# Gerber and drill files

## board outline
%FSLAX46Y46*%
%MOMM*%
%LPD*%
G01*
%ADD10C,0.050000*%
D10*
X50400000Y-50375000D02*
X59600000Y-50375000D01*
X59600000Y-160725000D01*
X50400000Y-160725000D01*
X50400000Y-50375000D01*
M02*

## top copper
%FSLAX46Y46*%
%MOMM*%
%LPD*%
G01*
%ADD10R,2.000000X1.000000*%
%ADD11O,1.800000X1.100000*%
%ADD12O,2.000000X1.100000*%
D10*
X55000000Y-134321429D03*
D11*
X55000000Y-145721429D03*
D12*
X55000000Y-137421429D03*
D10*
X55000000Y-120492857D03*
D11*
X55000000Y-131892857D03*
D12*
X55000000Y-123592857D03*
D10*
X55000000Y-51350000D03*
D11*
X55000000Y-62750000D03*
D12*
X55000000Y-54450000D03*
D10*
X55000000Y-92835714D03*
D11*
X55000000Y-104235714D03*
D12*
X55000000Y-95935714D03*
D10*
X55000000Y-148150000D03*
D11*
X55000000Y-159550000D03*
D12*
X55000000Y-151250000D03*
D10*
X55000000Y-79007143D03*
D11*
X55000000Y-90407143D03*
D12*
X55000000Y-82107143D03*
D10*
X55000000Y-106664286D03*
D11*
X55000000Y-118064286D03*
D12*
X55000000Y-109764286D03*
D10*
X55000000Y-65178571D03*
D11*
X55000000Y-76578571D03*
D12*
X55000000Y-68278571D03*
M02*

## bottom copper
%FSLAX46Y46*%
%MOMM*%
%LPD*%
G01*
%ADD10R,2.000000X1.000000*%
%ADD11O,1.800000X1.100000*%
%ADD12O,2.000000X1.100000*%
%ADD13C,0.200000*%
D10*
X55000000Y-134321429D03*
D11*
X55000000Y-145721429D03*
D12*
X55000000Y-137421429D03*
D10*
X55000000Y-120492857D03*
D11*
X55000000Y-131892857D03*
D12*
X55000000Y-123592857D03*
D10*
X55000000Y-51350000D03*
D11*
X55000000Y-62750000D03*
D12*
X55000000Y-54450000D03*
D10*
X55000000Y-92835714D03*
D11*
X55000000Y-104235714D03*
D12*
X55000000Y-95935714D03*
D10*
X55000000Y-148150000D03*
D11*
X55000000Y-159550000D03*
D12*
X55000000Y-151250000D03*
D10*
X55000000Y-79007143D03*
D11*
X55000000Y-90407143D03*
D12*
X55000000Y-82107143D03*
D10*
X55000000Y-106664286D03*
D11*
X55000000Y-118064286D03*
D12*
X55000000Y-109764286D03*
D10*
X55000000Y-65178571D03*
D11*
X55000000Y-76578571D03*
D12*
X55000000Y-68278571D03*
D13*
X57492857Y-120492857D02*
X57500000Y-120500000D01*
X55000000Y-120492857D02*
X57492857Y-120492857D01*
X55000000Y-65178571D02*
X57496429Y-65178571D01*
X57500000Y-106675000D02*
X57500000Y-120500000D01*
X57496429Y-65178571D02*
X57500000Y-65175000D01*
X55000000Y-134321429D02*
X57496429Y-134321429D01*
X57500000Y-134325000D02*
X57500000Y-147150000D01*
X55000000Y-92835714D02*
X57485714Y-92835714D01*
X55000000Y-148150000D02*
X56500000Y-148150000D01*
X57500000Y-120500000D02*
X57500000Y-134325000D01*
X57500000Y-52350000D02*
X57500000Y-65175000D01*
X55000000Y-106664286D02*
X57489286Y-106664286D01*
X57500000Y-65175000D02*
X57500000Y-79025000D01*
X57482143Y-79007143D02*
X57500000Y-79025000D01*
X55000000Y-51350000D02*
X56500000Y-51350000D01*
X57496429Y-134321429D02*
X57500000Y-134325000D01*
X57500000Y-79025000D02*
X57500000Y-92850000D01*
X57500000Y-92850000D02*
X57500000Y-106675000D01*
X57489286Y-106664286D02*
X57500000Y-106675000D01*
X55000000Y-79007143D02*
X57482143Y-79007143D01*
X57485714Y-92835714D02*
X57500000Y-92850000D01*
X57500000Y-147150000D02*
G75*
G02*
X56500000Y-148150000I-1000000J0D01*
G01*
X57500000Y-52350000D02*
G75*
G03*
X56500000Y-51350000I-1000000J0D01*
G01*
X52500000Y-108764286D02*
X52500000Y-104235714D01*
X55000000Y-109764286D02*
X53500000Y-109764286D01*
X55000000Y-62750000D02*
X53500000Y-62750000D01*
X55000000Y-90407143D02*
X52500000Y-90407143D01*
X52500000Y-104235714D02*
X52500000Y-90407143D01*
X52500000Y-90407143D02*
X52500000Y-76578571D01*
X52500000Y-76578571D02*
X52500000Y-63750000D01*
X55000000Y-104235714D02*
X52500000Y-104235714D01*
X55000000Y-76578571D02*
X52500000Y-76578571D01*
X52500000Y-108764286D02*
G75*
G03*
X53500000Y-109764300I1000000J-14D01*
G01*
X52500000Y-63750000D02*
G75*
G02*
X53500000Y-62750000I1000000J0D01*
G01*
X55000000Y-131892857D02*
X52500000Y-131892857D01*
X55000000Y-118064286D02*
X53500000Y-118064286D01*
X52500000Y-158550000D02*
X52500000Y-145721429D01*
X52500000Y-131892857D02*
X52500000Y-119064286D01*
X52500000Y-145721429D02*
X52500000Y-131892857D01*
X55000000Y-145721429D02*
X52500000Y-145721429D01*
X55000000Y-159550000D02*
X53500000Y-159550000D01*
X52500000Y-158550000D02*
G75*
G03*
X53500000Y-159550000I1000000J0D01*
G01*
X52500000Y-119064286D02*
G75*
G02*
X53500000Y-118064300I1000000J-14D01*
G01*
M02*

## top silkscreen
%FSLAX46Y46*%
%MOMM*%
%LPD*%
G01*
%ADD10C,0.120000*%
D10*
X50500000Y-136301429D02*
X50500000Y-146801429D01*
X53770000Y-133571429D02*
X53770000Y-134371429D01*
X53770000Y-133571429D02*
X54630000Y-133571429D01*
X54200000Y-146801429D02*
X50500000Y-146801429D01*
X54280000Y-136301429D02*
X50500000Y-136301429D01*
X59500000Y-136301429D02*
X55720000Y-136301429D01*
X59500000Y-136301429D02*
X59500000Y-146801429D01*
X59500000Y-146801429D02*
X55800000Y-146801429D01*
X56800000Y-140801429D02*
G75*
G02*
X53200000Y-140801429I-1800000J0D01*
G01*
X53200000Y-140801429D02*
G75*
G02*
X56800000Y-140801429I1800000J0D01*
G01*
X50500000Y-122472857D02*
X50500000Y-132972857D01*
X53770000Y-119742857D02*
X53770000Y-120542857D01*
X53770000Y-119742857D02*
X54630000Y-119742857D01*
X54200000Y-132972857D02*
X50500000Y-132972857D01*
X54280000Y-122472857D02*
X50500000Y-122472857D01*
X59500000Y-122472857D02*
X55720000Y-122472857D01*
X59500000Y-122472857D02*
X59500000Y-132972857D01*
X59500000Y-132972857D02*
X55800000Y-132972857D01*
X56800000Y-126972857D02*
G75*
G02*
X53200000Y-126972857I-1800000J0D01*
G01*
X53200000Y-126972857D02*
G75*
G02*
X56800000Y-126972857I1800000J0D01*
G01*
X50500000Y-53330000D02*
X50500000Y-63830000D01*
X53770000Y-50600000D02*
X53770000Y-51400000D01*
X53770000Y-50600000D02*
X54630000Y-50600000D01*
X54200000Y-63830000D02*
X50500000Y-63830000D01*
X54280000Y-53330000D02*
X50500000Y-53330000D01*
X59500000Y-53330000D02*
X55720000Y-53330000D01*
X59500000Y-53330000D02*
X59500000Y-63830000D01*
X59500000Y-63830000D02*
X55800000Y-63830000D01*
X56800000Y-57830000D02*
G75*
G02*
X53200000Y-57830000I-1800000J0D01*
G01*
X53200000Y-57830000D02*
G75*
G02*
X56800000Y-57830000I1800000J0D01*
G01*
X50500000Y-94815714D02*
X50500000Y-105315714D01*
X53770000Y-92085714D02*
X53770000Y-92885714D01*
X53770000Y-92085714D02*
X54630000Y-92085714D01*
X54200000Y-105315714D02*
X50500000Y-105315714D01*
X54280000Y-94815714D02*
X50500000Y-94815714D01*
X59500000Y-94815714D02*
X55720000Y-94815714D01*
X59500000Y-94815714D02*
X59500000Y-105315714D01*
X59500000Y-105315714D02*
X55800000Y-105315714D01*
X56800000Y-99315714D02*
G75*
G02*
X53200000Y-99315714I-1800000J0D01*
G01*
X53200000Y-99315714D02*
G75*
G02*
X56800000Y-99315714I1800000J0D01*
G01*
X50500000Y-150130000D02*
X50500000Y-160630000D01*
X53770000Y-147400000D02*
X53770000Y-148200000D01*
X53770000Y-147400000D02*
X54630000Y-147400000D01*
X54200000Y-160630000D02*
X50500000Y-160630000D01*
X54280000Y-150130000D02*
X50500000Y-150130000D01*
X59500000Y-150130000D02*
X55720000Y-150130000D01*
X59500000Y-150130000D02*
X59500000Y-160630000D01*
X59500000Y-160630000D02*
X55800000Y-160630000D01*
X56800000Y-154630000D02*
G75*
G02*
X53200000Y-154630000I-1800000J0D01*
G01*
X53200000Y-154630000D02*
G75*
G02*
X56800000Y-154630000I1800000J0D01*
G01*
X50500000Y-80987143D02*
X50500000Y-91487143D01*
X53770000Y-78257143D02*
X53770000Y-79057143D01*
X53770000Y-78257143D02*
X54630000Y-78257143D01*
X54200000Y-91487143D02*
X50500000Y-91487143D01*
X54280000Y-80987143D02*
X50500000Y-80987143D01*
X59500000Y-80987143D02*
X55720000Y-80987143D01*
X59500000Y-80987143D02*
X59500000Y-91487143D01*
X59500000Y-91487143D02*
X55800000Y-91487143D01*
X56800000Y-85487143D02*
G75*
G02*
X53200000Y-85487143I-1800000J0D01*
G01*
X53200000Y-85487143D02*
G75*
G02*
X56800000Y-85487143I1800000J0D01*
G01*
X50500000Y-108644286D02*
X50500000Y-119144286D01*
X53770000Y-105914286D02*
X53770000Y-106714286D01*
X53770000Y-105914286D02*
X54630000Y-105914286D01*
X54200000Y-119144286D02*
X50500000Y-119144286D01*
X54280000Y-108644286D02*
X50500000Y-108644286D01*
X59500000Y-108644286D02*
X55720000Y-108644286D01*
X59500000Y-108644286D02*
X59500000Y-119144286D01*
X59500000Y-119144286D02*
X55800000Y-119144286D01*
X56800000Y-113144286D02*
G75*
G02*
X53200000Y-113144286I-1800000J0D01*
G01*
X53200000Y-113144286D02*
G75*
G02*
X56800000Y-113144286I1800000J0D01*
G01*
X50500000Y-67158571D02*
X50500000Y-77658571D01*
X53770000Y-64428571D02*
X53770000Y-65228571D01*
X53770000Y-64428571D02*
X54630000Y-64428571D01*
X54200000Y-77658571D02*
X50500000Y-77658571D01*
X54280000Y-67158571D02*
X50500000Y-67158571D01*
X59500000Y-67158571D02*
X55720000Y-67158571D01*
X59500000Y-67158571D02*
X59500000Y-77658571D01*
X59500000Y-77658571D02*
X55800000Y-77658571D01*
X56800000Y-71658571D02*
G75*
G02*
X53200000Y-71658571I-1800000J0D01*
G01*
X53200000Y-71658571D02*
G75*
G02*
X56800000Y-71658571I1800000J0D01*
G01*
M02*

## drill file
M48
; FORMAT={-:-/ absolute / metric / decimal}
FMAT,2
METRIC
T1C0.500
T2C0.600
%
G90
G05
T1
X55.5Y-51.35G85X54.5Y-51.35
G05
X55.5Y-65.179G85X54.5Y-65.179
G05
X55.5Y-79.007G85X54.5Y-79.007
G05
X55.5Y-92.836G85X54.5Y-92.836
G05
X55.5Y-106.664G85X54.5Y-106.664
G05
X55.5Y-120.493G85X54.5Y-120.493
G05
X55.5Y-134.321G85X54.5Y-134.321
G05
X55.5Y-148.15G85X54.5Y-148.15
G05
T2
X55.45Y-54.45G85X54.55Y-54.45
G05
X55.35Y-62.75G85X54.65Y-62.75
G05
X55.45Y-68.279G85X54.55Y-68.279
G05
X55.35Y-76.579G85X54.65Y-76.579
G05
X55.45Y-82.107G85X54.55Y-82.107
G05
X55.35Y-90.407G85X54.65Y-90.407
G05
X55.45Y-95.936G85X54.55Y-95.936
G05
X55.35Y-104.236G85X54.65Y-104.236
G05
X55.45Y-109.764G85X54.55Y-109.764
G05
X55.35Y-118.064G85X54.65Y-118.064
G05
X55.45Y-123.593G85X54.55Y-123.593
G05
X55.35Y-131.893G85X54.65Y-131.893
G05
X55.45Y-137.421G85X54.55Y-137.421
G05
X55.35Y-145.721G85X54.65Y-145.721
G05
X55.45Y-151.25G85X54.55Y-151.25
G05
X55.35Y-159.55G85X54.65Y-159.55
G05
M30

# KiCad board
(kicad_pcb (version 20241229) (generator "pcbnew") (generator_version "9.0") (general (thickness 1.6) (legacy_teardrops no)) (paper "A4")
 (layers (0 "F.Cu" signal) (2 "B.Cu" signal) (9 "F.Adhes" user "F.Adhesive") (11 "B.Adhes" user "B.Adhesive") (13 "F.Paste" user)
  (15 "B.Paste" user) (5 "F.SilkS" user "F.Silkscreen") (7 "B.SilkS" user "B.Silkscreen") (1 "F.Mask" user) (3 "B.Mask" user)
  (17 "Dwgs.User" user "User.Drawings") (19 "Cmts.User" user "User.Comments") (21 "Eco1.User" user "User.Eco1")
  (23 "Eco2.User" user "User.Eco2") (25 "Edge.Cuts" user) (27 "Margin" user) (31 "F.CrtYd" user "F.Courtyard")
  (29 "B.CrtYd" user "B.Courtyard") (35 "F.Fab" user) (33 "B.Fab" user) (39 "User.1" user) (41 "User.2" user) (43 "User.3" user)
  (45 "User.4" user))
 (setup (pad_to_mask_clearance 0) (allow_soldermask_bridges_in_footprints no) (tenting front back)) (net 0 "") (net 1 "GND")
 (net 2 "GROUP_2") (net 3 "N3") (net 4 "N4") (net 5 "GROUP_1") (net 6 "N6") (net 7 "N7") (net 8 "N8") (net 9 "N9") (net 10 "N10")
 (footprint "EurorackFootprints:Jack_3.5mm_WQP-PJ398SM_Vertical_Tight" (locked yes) (layer "F.Cu") (at 55 134.321429)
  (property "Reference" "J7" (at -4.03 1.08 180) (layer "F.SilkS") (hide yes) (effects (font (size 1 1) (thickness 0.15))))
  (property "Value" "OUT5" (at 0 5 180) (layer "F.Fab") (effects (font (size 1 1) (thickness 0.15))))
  (fp_line (start -4.5 1.98) (end -4.5 12.48) (stroke (width 0.12) (type solid)) (layer "F.SilkS"))
  (fp_line (start -1.23 -0.75) (end -1.23 0.05) (stroke (width 0.12) (type solid)) (layer "F.SilkS"))
  (fp_line (start -1.23 -0.75) (end -0.37 -0.75) (stroke (width 0.12) (type solid)) (layer "F.SilkS"))
  (fp_line (start -0.8 12.48) (end -4.5 12.48) (stroke (width 0.12) (type solid)) (layer "F.SilkS"))
  (fp_line (start -0.72 1.98) (end -4.5 1.98) (stroke (width 0.12) (type solid)) (layer "F.SilkS"))
  (fp_line (start 4.5 1.98) (end 0.72 1.98) (stroke (width 0.12) (type solid)) (layer "F.SilkS"))
  (fp_line (start 4.5 1.98) (end 4.5 12.48) (stroke (width 0.12) (type solid)) (layer "F.SilkS"))
  (fp_line (start 4.5 12.48) (end 0.8 12.48) (stroke (width 0.12) (type solid)) (layer "F.SilkS"))
  (fp_circle (center 0 6.48) (end 1.8 6.48) (stroke (width 0.12) (type solid)) (fill no) (layer "F.SilkS"))
  (pad "S" thru_hole rect (at 0 0 180) (size 2 1) (drill oval 1.5 0.5) (layers "*.Cu" "*.Mask") (remove_unused_layers no) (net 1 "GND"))
  (pad "T" thru_hole oval (at 0 11.4 180) (size 1.8 1.1) (drill oval 1.3 0.6) (layers "*.Cu" "*.Mask") (remove_unused_layers no)
   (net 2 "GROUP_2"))
  (pad "TN" thru_hole oval (at 0 3.1 180) (size 2 1.1) (drill oval 1.5 0.6) (layers "*.Cu" "*.Mask") (remove_unused_layers no) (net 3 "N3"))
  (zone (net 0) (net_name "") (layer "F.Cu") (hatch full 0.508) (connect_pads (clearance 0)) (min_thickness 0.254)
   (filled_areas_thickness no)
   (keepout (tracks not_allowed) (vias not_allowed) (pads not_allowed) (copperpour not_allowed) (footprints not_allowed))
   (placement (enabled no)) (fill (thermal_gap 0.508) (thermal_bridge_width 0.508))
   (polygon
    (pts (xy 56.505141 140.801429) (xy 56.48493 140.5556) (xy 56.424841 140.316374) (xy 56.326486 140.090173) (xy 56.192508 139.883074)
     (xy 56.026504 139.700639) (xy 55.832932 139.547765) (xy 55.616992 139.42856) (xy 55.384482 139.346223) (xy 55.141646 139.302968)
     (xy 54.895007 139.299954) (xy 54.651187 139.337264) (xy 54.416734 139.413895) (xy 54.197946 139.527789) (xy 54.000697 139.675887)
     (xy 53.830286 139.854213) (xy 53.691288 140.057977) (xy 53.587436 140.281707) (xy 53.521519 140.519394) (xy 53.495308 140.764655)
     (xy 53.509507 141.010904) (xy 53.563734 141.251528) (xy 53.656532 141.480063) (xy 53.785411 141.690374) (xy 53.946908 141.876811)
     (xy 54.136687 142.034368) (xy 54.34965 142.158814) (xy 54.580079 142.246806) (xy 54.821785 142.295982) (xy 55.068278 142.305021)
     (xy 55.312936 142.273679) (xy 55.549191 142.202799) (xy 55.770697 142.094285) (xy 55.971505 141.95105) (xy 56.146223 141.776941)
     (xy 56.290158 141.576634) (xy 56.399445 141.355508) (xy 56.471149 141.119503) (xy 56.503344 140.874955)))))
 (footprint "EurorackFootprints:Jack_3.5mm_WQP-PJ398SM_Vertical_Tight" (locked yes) (layer "F.Cu") (at 55 120.492857)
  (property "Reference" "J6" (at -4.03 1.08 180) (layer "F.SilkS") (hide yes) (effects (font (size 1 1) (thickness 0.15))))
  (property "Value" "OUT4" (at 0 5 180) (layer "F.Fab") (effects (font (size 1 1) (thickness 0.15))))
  (fp_line (start -4.5 1.98) (end -4.5 12.48) (stroke (width 0.12) (type solid)) (layer "F.SilkS"))
  (fp_line (start -1.23 -0.75) (end -1.23 0.05) (stroke (width 0.12) (type solid)) (layer "F.SilkS"))
  (fp_line (start -1.23 -0.75) (end -0.37 -0.75) (stroke (width 0.12) (type solid)) (layer "F.SilkS"))
  (fp_line (start -0.8 12.48) (end -4.5 12.48) (stroke (width 0.12) (type solid)) (layer "F.SilkS"))
  (fp_line (start -0.72 1.98) (end -4.5 1.98) (stroke (width 0.12) (type solid)) (layer "F.SilkS"))
  (fp_line (start 4.5 1.98) (end 0.72 1.98) (stroke (width 0.12) (type solid)) (layer "F.SilkS"))
  (fp_line (start 4.5 1.98) (end 4.5 12.48) (stroke (width 0.12) (type solid)) (layer "F.SilkS"))
  (fp_line (start 4.5 12.48) (end 0.8 12.48) (stroke (width 0.12) (type solid)) (layer "F.SilkS"))
  (fp_circle (center 0 6.48) (end 1.8 6.48) (stroke (width 0.12) (type solid)) (fill no) (layer "F.SilkS"))
  (pad "S" thru_hole rect (at 0 0 180) (size 2 1) (drill oval 1.5 0.5) (layers "*.Cu" "*.Mask") (remove_unused_layers no) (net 1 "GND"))
  (pad "T" thru_hole oval (at 0 11.4 180) (size 1.8 1.1) (drill oval 1.3 0.6) (layers "*.Cu" "*.Mask") (remove_unused_layers no)
   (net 2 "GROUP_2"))
  (pad "TN" thru_hole oval (at 0 3.1 180) (size 2 1.1) (drill oval 1.5 0.6) (layers "*.Cu" "*.Mask") (remove_unused_layers no) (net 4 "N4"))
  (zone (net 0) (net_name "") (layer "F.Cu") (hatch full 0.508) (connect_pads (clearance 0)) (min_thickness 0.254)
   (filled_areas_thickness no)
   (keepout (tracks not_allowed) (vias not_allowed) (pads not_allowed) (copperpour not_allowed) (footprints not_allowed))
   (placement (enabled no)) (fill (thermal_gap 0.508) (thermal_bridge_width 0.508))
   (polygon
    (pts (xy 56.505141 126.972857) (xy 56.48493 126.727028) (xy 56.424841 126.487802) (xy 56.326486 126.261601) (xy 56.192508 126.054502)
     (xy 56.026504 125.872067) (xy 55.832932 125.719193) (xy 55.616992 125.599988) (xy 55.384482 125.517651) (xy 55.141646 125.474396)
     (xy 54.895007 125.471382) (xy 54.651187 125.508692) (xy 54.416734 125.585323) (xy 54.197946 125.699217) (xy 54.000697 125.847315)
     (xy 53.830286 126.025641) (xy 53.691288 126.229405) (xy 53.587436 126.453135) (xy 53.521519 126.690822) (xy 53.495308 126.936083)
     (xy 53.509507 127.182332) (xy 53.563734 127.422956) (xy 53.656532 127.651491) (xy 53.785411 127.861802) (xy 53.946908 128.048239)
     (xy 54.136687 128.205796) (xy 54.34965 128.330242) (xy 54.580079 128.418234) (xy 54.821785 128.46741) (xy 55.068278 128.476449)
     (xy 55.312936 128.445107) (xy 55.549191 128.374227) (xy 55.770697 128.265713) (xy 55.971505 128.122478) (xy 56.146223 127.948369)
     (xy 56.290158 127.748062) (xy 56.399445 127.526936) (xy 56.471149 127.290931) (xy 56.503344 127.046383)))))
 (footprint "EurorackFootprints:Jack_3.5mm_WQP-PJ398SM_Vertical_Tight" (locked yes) (layer "F.Cu") (at 55 51.35)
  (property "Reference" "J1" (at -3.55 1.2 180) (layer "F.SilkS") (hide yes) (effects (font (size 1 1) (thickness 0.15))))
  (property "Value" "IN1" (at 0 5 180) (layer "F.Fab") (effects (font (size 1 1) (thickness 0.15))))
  (fp_line (start -4.5 1.98) (end -4.5 12.48) (stroke (width 0.12) (type solid)) (layer "F.SilkS"))
  (fp_line (start -1.23 -0.75) (end -1.23 0.05) (stroke (width 0.12) (type solid)) (layer "F.SilkS"))
  (fp_line (start -1.23 -0.75) (end -0.37 -0.75) (stroke (width 0.12) (type solid)) (layer "F.SilkS"))
  (fp_line (start -0.8 12.48) (end -4.5 12.48) (stroke (width 0.12) (type solid)) (layer "F.SilkS"))
  (fp_line (start -0.72 1.98) (end -4.5 1.98) (stroke (width 0.12) (type solid)) (layer "F.SilkS"))
  (fp_line (start 4.5 1.98) (end 0.72 1.98) (stroke (width 0.12) (type solid)) (layer "F.SilkS"))
  (fp_line (start 4.5 1.98) (end 4.5 12.48) (stroke (width 0.12) (type solid)) (layer "F.SilkS"))
  (fp_line (start 4.5 12.48) (end 0.8 12.48) (stroke (width 0.12) (type solid)) (layer "F.SilkS"))
  (fp_circle (center 0 6.48) (end 1.8 6.48) (stroke (width 0.12) (type solid)) (fill no) (layer "F.SilkS"))
  (pad "S" thru_hole rect (at 0 0 180) (size 2 1) (drill oval 1.5 0.5) (layers "*.Cu" "*.Mask") (remove_unused_layers no) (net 1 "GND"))
  (pad "T" thru_hole oval (at 0 11.4 180) (size 1.8 1.1) (drill oval 1.3 0.6) (layers "*.Cu" "*.Mask") (remove_unused_layers no)
   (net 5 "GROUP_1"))
  (pad "TN" thru_hole oval (at 0 3.1 180) (size 2 1.1) (drill oval 1.5 0.6) (layers "*.Cu" "*.Mask") (remove_unused_layers no) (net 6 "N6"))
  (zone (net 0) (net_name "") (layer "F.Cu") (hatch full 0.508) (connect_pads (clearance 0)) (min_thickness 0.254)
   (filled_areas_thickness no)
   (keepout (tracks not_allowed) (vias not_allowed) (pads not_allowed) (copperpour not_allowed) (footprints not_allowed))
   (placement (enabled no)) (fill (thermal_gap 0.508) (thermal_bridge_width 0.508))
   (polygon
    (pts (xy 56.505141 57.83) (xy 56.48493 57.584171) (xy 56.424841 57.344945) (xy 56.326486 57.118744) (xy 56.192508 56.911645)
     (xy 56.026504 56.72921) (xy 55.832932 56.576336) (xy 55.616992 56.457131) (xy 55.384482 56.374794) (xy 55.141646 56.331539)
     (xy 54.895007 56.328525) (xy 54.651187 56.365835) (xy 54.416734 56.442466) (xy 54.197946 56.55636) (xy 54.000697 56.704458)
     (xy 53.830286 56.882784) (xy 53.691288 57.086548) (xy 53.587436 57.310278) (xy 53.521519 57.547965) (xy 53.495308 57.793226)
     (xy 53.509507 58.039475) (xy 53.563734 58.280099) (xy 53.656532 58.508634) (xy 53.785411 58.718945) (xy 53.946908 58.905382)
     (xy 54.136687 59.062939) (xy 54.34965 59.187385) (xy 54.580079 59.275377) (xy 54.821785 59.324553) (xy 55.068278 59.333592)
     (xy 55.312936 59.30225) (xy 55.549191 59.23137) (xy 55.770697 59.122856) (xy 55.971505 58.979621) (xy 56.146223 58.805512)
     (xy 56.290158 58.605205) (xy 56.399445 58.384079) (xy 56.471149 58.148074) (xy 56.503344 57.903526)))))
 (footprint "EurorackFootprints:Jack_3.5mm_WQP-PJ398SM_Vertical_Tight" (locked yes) (layer "F.Cu") (at 55 92.835714)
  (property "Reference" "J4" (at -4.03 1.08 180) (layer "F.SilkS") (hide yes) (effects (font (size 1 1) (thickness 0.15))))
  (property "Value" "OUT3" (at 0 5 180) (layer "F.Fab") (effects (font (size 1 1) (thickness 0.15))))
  (fp_line (start -4.5 1.98) (end -4.5 12.48) (stroke (width 0.12) (type solid)) (layer "F.SilkS"))
  (fp_line (start -1.23 -0.75) (end -1.23 0.05) (stroke (width 0.12) (type solid)) (layer "F.SilkS"))
  (fp_line (start -1.23 -0.75) (end -0.37 -0.75) (stroke (width 0.12) (type solid)) (layer "F.SilkS"))
  (fp_line (start -0.8 12.48) (end -4.5 12.48) (stroke (width 0.12) (type solid)) (layer "F.SilkS"))
  (fp_line (start -0.72 1.98) (end -4.5 1.98) (stroke (width 0.12) (type solid)) (layer "F.SilkS"))
  (fp_line (start 4.5 1.98) (end 0.72 1.98) (stroke (width 0.12) (type solid)) (layer "F.SilkS"))
  (fp_line (start 4.5 1.98) (end 4.5 12.48) (stroke (width 0.12) (type solid)) (layer "F.SilkS"))
  (fp_line (start 4.5 12.48) (end 0.8 12.48) (stroke (width 0.12) (type solid)) (layer "F.SilkS"))
  (fp_circle (center 0 6.48) (end 1.8 6.48) (stroke (width 0.12) (type solid)) (fill no) (layer "F.SilkS"))
  (pad "S" thru_hole rect (at 0 0 180) (size 2 1) (drill oval 1.5 0.5) (layers "*.Cu" "*.Mask") (remove_unused_layers no) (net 1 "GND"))
  (pad "T" thru_hole oval (at 0 11.4 180) (size 1.8 1.1) (drill oval 1.3 0.6) (layers "*.Cu" "*.Mask") (remove_unused_layers no)
   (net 5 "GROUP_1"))
  (pad "TN" thru_hole oval (at 0 3.1 180) (size 2 1.1) (drill oval 1.5 0.6) (layers "*.Cu" "*.Mask") (remove_unused_layers no) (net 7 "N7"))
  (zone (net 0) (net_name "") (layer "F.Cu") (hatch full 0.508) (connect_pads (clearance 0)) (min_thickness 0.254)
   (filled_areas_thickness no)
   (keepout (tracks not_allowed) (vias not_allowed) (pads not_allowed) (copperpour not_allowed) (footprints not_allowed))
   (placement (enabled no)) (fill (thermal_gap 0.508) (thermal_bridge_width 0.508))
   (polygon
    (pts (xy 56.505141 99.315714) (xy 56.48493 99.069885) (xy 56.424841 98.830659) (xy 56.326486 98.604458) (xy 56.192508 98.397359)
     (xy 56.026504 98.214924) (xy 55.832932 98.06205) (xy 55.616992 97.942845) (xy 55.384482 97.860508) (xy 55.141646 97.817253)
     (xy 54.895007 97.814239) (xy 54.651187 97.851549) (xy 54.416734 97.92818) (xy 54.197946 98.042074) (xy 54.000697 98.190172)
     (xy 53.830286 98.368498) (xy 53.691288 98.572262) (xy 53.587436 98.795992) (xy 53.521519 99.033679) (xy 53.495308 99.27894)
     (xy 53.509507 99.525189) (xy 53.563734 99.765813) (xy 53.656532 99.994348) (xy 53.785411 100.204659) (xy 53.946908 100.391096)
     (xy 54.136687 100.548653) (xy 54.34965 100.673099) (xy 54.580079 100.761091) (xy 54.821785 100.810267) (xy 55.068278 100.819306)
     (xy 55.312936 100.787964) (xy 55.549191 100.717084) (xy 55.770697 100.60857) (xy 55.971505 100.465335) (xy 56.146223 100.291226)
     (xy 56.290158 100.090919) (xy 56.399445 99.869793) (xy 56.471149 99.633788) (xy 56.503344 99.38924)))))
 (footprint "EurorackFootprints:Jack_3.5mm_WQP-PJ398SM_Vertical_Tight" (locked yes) (layer "F.Cu") (at 55 148.15)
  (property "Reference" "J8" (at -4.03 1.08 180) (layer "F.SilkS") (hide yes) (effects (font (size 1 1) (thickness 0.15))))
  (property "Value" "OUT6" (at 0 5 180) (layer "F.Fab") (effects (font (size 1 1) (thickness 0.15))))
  (fp_line (start -4.5 1.98) (end -4.5 12.48) (stroke (width 0.12) (type solid)) (layer "F.SilkS"))
  (fp_line (start -1.23 -0.75) (end -1.23 0.05) (stroke (width 0.12) (type solid)) (layer "F.SilkS"))
  (fp_line (start -1.23 -0.75) (end -0.37 -0.75) (stroke (width 0.12) (type solid)) (layer "F.SilkS"))
  (fp_line (start -0.8 12.48) (end -4.5 12.48) (stroke (width 0.12) (type solid)) (layer "F.SilkS"))
  (fp_line (start -0.72 1.98) (end -4.5 1.98) (stroke (width 0.12) (type solid)) (layer "F.SilkS"))
  (fp_line (start 4.5 1.98) (end 0.72 1.98) (stroke (width 0.12) (type solid)) (layer "F.SilkS"))
  (fp_line (start 4.5 1.98) (end 4.5 12.48) (stroke (width 0.12) (type solid)) (layer "F.SilkS"))
  (fp_line (start 4.5 12.48) (end 0.8 12.48) (stroke (width 0.12) (type solid)) (layer "F.SilkS"))
  (fp_circle (center 0 6.48) (end 1.8 6.48) (stroke (width 0.12) (type solid)) (fill no) (layer "F.SilkS"))
  (pad "S" thru_hole rect (at 0 0 180) (size 2 1) (drill oval 1.5 0.5) (layers "*.Cu" "*.Mask") (remove_unused_layers no) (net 1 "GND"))
  (pad "T" thru_hole oval (at 0 11.4 180) (size 1.8 1.1) (drill oval 1.3 0.6) (layers "*.Cu" "*.Mask") (remove_unused_layers no)
   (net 2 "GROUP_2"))
  (pad "TN" thru_hole oval (at 0 3.1 180) (size 2 1.1) (drill oval 1.5 0.6) (layers "*.Cu" "*.Mask") (remove_unused_layers no) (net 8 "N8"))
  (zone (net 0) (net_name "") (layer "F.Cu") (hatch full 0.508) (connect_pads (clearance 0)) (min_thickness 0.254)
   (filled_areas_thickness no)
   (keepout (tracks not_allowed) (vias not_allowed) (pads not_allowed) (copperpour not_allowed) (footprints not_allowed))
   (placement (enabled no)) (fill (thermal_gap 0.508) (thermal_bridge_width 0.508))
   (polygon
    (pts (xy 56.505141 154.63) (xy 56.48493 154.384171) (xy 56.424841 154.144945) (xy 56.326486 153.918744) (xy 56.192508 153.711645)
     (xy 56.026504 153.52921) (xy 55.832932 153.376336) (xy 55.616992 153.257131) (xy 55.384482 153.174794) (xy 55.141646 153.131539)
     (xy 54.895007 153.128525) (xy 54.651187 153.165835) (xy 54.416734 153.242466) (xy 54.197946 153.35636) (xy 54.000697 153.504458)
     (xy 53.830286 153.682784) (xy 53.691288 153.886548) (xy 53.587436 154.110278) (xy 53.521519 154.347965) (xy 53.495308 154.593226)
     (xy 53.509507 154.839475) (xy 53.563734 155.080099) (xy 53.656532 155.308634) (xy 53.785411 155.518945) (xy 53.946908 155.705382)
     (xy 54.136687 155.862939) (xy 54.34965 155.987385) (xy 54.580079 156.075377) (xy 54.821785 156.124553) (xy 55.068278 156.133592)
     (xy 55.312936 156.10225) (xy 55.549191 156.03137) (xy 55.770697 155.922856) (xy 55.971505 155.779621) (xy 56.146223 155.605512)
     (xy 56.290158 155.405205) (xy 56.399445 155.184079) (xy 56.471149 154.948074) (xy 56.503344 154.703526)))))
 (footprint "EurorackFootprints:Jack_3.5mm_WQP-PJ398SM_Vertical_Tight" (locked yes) (layer "F.Cu") (at 55 79.007143)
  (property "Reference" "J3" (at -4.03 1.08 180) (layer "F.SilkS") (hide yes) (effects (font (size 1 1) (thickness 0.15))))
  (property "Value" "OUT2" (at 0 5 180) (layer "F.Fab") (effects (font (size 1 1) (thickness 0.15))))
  (fp_line (start -4.5 1.98) (end -4.5 12.48) (stroke (width 0.12) (type solid)) (layer "F.SilkS"))
  (fp_line (start -1.23 -0.75) (end -1.23 0.05) (stroke (width 0.12) (type solid)) (layer "F.SilkS"))
  (fp_line (start -1.23 -0.75) (end -0.37 -0.75) (stroke (width 0.12) (type solid)) (layer "F.SilkS"))
  (fp_line (start -0.8 12.48) (end -4.5 12.48) (stroke (width 0.12) (type solid)) (layer "F.SilkS"))
  (fp_line (start -0.72 1.98) (end -4.5 1.98) (stroke (width 0.12) (type solid)) (layer "F.SilkS"))
  (fp_line (start 4.5 1.98) (end 0.72 1.98) (stroke (width 0.12) (type solid)) (layer "F.SilkS"))
  (fp_line (start 4.5 1.98) (end 4.5 12.48) (stroke (width 0.12) (type solid)) (layer "F.SilkS"))
  (fp_line (start 4.5 12.48) (end 0.8 12.48) (stroke (width 0.12) (type solid)) (layer "F.SilkS"))
  (fp_circle (center 0 6.48) (end 1.8 6.48) (stroke (width 0.12) (type solid)) (fill no) (layer "F.SilkS"))
  (pad "S" thru_hole rect (at 0 0 180) (size 2 1) (drill oval 1.5 0.5) (layers "*.Cu" "*.Mask") (remove_unused_layers no) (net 1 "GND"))
  (pad "T" thru_hole oval (at 0 11.4 180) (size 1.8 1.1) (drill oval 1.3 0.6) (layers "*.Cu" "*.Mask") (remove_unused_layers no)
   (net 5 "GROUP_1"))
  (pad "TN" thru_hole oval (at 0 3.1 180) (size 2 1.1) (drill oval 1.5 0.6) (layers "*.Cu" "*.Mask") (remove_unused_layers no) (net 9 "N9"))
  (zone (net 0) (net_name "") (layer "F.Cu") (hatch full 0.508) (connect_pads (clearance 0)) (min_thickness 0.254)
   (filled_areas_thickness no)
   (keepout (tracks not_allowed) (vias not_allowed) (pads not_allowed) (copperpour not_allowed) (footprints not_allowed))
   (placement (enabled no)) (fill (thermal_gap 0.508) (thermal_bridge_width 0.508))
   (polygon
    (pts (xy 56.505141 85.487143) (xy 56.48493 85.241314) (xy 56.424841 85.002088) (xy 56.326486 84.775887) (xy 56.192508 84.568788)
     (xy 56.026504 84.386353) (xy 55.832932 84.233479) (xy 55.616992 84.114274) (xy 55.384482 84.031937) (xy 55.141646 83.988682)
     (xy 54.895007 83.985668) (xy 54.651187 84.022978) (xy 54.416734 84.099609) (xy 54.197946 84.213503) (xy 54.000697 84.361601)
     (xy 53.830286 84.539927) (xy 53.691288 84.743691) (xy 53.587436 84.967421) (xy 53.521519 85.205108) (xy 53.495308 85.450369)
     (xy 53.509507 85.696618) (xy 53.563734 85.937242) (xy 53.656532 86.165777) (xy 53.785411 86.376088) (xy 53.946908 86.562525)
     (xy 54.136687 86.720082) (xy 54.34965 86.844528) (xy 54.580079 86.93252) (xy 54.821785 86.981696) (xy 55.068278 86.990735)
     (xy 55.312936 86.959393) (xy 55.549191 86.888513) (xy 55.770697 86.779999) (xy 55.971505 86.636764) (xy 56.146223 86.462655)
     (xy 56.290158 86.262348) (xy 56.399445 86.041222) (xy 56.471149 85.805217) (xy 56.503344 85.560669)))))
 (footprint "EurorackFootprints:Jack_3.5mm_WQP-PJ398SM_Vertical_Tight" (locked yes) (layer "F.Cu") (at 55 106.664286)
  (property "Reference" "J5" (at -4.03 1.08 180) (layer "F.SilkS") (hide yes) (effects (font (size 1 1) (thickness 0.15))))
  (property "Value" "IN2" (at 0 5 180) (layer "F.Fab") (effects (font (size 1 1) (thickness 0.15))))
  (fp_line (start -4.5 1.98) (end -4.5 12.48) (stroke (width 0.12) (type solid)) (layer "F.SilkS"))
  (fp_line (start -1.23 -0.75) (end -1.23 0.05) (stroke (width 0.12) (type solid)) (layer "F.SilkS"))
  (fp_line (start -1.23 -0.75) (end -0.37 -0.75) (stroke (width 0.12) (type solid)) (layer "F.SilkS"))
  (fp_line (start -0.8 12.48) (end -4.5 12.48) (stroke (width 0.12) (type solid)) (layer "F.SilkS"))
  (fp_line (start -0.72 1.98) (end -4.5 1.98) (stroke (width 0.12) (type solid)) (layer "F.SilkS"))
  (fp_line (start 4.5 1.98) (end 0.72 1.98) (stroke (width 0.12) (type solid)) (layer "F.SilkS"))
  (fp_line (start 4.5 1.98) (end 4.5 12.48) (stroke (width 0.12) (type solid)) (layer "F.SilkS"))
  (fp_line (start 4.5 12.48) (end 0.8 12.48) (stroke (width 0.12) (type solid)) (layer "F.SilkS"))
  (fp_circle (center 0 6.48) (end 1.8 6.48) (stroke (width 0.12) (type solid)) (fill no) (layer "F.SilkS"))
  (pad "S" thru_hole rect (at 0 0 180) (size 2 1) (drill oval 1.5 0.5) (layers "*.Cu" "*.Mask") (remove_unused_layers no) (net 1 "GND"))
  (pad "T" thru_hole oval (at 0 11.4 180) (size 1.8 1.1) (drill oval 1.3 0.6) (layers "*.Cu" "*.Mask") (remove_unused_layers no)
   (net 2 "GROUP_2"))
  (pad "TN" thru_hole oval (at 0 3.1 180) (size 2 1.1) (drill oval 1.5 0.6) (layers "*.Cu" "*.Mask") (remove_unused_layers no)
   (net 5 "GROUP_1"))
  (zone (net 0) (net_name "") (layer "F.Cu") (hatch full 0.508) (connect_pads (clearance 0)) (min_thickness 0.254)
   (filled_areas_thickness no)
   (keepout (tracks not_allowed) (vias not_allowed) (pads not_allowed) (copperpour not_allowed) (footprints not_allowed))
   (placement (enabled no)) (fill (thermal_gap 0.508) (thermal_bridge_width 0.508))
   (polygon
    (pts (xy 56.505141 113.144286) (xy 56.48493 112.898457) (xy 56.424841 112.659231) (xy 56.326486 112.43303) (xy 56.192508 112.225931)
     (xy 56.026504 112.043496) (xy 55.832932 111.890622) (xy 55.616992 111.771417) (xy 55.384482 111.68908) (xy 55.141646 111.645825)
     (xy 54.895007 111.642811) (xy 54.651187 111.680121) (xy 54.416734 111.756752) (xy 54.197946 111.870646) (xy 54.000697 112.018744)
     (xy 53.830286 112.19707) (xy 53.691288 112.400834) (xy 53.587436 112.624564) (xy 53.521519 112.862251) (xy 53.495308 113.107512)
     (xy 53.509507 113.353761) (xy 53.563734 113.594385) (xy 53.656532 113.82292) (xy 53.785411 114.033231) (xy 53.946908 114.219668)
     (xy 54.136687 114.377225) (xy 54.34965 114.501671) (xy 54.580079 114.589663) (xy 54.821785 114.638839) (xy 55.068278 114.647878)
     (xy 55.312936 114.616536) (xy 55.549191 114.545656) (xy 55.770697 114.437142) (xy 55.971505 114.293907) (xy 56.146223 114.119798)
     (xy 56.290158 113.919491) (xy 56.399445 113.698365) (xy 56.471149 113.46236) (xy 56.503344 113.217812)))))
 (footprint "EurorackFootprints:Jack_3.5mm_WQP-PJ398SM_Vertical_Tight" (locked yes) (layer "F.Cu") (at 55 65.178571)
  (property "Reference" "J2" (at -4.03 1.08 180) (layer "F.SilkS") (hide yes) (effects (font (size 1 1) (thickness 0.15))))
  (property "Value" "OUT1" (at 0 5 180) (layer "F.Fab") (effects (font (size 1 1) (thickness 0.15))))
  (fp_line (start -4.5 1.98) (end -4.5 12.48) (stroke (width 0.12) (type solid)) (layer "F.SilkS"))
  (fp_line (start -1.23 -0.75) (end -1.23 0.05) (stroke (width 0.12) (type solid)) (layer "F.SilkS"))
  (fp_line (start -1.23 -0.75) (end -0.37 -0.75) (stroke (width 0.12) (type solid)) (layer "F.SilkS"))
  (fp_line (start -0.8 12.48) (end -4.5 12.48) (stroke (width 0.12) (type solid)) (layer "F.SilkS"))
  (fp_line (start -0.72 1.98) (end -4.5 1.98) (stroke (width 0.12) (type solid)) (layer "F.SilkS"))
  (fp_line (start 4.5 1.98) (end 0.72 1.98) (stroke (width 0.12) (type solid)) (layer "F.SilkS"))
  (fp_line (start 4.5 1.98) (end 4.5 12.48) (stroke (width 0.12) (type solid)) (layer "F.SilkS"))
  (fp_line (start 4.5 12.48) (end 0.8 12.48) (stroke (width 0.12) (type solid)) (layer "F.SilkS"))
  (fp_circle (center 0 6.48) (end 1.8 6.48) (stroke (width 0.12) (type solid)) (fill no) (layer "F.SilkS"))
  (pad "S" thru_hole rect (at 0 0 180) (size 2 1) (drill oval 1.5 0.5) (layers "*.Cu" "*.Mask") (remove_unused_layers no) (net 1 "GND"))
  (pad "T" thru_hole oval (at 0 11.4 180) (size 1.8 1.1) (drill oval 1.3 0.6) (layers "*.Cu" "*.Mask") (remove_unused_layers no)
   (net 5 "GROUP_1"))
  (pad "TN" thru_hole oval (at 0 3.1 180) (size 2 1.1) (drill oval 1.5 0.6) (layers "*.Cu" "*.Mask") (remove_unused_layers no)
   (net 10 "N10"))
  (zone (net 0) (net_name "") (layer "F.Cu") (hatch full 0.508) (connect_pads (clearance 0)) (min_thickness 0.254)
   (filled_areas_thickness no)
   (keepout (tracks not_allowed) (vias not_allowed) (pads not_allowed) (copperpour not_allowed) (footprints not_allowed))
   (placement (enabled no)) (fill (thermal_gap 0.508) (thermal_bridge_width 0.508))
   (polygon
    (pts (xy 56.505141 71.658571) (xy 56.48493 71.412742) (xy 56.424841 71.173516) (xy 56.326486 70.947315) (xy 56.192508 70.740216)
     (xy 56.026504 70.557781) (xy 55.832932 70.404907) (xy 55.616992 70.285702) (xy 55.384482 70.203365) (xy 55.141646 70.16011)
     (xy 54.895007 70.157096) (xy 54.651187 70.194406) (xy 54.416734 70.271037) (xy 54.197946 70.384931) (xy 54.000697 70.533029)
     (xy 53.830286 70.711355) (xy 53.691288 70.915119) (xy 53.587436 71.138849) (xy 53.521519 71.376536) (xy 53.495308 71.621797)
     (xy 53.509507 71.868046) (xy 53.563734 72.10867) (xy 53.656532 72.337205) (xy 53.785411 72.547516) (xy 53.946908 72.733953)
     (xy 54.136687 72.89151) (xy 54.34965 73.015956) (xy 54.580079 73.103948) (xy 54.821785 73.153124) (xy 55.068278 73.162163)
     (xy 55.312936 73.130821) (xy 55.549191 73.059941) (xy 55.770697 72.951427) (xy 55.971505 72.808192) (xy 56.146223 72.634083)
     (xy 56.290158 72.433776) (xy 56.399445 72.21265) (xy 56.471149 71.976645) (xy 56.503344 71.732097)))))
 (gr_rect (start 50.4 50.375) (end 59.6 160.725) (stroke (width 0.05) (type default)) (fill no) (layer "Edge.Cuts"))
 (segment (start 57.492857 120.492857) (end 57.5 120.5) (width 0.2) (layer "B.Cu") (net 1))
 (segment (start 55 120.492857) (end 57.492857 120.492857) (width 0.2) (layer "B.Cu") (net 1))
 (segment (start 55 65.178571) (end 57.496429 65.178571) (width 0.2) (layer "B.Cu") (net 1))
 (segment (start 57.5 106.675) (end 57.5 120.5) (width 0.2) (layer "B.Cu") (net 1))
 (segment (start 57.496429 65.178571) (end 57.5 65.175) (width 0.2) (layer "B.Cu") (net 1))
 (segment (start 55 134.321429) (end 57.496429 134.321429) (width 0.2) (layer "B.Cu") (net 1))
 (segment (start 57.5 134.325) (end 57.5 147.15) (width 0.2) (layer "B.Cu") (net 1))
 (segment (start 55 92.835714) (end 57.485714 92.835714) (width 0.2) (layer "B.Cu") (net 1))
 (segment (start 55 148.15) (end 56.5 148.15) (width 0.2) (layer "B.Cu") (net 1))
 (segment (start 57.5 120.5) (end 57.5 134.325) (width 0.2) (layer "B.Cu") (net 1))
 (segment (start 57.5 52.35) (end 57.5 65.175) (width 0.2) (layer "B.Cu") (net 1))
 (segment (start 55 106.664286) (end 57.489286 106.664286) (width 0.2) (layer "B.Cu") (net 1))
 (segment (start 57.5 65.175) (end 57.5 79.025) (width 0.2) (layer "B.Cu") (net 1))
 (segment (start 57.482143 79.007143) (end 57.5 79.025) (width 0.2) (layer "B.Cu") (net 1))
 (segment (start 55 51.35) (end 56.5 51.35) (width 0.2) (layer "B.Cu") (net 1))
 (segment (start 57.496429 134.321429) (end 57.5 134.325) (width 0.2) (layer "B.Cu") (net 1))
 (segment (start 57.5 79.025) (end 57.5 92.85) (width 0.2) (layer "B.Cu") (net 1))
 (segment (start 57.5 92.85) (end 57.5 106.675) (width 0.2) (layer "B.Cu") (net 1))
 (segment (start 57.489286 106.664286) (end 57.5 106.675) (width 0.2) (layer "B.Cu") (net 1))
 (segment (start 55 79.007143) (end 57.482143 79.007143) (width 0.2) (layer "B.Cu") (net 1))
 (segment (start 57.485714 92.835714) (end 57.5 92.85) (width 0.2) (layer "B.Cu") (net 1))
 (arc (start 57.5 147.15) (mid 57.207107 147.857107) (end 56.5 148.15) (width 0.2) (layer "B.Cu") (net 1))
 (arc (start 57.5 52.35) (mid 57.207107 51.642893) (end 56.5 51.35) (width 0.2) (layer "B.Cu") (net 1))
 (segment (start 52.5 108.764286) (end 52.5 104.235714) (width 0.2) (layer "B.Cu") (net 5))
 (segment (start 55 109.764286) (end 53.5 109.764286) (width 0.2) (layer "B.Cu") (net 5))
 (segment (start 55 62.75) (end 53.5 62.75) (width 0.2) (layer "B.Cu") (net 5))
 (segment (start 55 90.407143) (end 52.5 90.407143) (width 0.2) (layer "B.Cu") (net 5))
 (segment (start 52.5 104.235714) (end 52.5 90.407143) (width 0.2) (layer "B.Cu") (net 5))
 (segment (start 52.5 90.407143) (end 52.5 76.578571) (width 0.2) (layer "B.Cu") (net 5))
 (segment (start 52.5 76.578571) (end 52.5 63.75) (width 0.2) (layer "B.Cu") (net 5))
 (segment (start 55 104.235714) (end 52.5 104.235714) (width 0.2) (layer "B.Cu") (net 5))
 (segment (start 55 76.578571) (end 52.5 76.578571) (width 0.2) (layer "B.Cu") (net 5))
 (arc (start 52.5 108.764286) (mid 52.792893 109.471393) (end 53.5 109.764286) (width 0.2) (layer "B.Cu") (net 5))
 (arc (start 52.5 63.75) (mid 52.792893 63.042893) (end 53.5 62.75) (width 0.2) (layer "B.Cu") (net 5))
 (segment (start 55 131.892857) (end 52.5 131.892857) (width 0.2) (layer "B.Cu") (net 2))
 (segment (start 55 118.064286) (end 53.5 118.064286) (width 0.2) (layer "B.Cu") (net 2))
 (segment (start 52.5 158.55) (end 52.5 145.721429) (width 0.2) (layer "B.Cu") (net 2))
 (segment (start 52.5 131.892857) (end 52.5 119.064286) (width 0.2) (layer "B.Cu") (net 2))
 (segment (start 52.5 145.721429) (end 52.5 131.892857) (width 0.2) (layer "B.Cu") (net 2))
 (segment (start 55 145.721429) (end 52.5 145.721429) (width 0.2) (layer "B.Cu") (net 2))
 (segment (start 55 159.55) (end 53.5 159.55) (width 0.2) (layer "B.Cu") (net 2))
 (arc (start 52.5 158.55) (mid 52.792893 159.257107) (end 53.5 159.55) (width 0.2) (layer "B.Cu") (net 2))
 (arc (start 52.5 119.064286) (mid 52.792893 118.357179) (end 53.5 118.064286) (width 0.2) (layer "B.Cu") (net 2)))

